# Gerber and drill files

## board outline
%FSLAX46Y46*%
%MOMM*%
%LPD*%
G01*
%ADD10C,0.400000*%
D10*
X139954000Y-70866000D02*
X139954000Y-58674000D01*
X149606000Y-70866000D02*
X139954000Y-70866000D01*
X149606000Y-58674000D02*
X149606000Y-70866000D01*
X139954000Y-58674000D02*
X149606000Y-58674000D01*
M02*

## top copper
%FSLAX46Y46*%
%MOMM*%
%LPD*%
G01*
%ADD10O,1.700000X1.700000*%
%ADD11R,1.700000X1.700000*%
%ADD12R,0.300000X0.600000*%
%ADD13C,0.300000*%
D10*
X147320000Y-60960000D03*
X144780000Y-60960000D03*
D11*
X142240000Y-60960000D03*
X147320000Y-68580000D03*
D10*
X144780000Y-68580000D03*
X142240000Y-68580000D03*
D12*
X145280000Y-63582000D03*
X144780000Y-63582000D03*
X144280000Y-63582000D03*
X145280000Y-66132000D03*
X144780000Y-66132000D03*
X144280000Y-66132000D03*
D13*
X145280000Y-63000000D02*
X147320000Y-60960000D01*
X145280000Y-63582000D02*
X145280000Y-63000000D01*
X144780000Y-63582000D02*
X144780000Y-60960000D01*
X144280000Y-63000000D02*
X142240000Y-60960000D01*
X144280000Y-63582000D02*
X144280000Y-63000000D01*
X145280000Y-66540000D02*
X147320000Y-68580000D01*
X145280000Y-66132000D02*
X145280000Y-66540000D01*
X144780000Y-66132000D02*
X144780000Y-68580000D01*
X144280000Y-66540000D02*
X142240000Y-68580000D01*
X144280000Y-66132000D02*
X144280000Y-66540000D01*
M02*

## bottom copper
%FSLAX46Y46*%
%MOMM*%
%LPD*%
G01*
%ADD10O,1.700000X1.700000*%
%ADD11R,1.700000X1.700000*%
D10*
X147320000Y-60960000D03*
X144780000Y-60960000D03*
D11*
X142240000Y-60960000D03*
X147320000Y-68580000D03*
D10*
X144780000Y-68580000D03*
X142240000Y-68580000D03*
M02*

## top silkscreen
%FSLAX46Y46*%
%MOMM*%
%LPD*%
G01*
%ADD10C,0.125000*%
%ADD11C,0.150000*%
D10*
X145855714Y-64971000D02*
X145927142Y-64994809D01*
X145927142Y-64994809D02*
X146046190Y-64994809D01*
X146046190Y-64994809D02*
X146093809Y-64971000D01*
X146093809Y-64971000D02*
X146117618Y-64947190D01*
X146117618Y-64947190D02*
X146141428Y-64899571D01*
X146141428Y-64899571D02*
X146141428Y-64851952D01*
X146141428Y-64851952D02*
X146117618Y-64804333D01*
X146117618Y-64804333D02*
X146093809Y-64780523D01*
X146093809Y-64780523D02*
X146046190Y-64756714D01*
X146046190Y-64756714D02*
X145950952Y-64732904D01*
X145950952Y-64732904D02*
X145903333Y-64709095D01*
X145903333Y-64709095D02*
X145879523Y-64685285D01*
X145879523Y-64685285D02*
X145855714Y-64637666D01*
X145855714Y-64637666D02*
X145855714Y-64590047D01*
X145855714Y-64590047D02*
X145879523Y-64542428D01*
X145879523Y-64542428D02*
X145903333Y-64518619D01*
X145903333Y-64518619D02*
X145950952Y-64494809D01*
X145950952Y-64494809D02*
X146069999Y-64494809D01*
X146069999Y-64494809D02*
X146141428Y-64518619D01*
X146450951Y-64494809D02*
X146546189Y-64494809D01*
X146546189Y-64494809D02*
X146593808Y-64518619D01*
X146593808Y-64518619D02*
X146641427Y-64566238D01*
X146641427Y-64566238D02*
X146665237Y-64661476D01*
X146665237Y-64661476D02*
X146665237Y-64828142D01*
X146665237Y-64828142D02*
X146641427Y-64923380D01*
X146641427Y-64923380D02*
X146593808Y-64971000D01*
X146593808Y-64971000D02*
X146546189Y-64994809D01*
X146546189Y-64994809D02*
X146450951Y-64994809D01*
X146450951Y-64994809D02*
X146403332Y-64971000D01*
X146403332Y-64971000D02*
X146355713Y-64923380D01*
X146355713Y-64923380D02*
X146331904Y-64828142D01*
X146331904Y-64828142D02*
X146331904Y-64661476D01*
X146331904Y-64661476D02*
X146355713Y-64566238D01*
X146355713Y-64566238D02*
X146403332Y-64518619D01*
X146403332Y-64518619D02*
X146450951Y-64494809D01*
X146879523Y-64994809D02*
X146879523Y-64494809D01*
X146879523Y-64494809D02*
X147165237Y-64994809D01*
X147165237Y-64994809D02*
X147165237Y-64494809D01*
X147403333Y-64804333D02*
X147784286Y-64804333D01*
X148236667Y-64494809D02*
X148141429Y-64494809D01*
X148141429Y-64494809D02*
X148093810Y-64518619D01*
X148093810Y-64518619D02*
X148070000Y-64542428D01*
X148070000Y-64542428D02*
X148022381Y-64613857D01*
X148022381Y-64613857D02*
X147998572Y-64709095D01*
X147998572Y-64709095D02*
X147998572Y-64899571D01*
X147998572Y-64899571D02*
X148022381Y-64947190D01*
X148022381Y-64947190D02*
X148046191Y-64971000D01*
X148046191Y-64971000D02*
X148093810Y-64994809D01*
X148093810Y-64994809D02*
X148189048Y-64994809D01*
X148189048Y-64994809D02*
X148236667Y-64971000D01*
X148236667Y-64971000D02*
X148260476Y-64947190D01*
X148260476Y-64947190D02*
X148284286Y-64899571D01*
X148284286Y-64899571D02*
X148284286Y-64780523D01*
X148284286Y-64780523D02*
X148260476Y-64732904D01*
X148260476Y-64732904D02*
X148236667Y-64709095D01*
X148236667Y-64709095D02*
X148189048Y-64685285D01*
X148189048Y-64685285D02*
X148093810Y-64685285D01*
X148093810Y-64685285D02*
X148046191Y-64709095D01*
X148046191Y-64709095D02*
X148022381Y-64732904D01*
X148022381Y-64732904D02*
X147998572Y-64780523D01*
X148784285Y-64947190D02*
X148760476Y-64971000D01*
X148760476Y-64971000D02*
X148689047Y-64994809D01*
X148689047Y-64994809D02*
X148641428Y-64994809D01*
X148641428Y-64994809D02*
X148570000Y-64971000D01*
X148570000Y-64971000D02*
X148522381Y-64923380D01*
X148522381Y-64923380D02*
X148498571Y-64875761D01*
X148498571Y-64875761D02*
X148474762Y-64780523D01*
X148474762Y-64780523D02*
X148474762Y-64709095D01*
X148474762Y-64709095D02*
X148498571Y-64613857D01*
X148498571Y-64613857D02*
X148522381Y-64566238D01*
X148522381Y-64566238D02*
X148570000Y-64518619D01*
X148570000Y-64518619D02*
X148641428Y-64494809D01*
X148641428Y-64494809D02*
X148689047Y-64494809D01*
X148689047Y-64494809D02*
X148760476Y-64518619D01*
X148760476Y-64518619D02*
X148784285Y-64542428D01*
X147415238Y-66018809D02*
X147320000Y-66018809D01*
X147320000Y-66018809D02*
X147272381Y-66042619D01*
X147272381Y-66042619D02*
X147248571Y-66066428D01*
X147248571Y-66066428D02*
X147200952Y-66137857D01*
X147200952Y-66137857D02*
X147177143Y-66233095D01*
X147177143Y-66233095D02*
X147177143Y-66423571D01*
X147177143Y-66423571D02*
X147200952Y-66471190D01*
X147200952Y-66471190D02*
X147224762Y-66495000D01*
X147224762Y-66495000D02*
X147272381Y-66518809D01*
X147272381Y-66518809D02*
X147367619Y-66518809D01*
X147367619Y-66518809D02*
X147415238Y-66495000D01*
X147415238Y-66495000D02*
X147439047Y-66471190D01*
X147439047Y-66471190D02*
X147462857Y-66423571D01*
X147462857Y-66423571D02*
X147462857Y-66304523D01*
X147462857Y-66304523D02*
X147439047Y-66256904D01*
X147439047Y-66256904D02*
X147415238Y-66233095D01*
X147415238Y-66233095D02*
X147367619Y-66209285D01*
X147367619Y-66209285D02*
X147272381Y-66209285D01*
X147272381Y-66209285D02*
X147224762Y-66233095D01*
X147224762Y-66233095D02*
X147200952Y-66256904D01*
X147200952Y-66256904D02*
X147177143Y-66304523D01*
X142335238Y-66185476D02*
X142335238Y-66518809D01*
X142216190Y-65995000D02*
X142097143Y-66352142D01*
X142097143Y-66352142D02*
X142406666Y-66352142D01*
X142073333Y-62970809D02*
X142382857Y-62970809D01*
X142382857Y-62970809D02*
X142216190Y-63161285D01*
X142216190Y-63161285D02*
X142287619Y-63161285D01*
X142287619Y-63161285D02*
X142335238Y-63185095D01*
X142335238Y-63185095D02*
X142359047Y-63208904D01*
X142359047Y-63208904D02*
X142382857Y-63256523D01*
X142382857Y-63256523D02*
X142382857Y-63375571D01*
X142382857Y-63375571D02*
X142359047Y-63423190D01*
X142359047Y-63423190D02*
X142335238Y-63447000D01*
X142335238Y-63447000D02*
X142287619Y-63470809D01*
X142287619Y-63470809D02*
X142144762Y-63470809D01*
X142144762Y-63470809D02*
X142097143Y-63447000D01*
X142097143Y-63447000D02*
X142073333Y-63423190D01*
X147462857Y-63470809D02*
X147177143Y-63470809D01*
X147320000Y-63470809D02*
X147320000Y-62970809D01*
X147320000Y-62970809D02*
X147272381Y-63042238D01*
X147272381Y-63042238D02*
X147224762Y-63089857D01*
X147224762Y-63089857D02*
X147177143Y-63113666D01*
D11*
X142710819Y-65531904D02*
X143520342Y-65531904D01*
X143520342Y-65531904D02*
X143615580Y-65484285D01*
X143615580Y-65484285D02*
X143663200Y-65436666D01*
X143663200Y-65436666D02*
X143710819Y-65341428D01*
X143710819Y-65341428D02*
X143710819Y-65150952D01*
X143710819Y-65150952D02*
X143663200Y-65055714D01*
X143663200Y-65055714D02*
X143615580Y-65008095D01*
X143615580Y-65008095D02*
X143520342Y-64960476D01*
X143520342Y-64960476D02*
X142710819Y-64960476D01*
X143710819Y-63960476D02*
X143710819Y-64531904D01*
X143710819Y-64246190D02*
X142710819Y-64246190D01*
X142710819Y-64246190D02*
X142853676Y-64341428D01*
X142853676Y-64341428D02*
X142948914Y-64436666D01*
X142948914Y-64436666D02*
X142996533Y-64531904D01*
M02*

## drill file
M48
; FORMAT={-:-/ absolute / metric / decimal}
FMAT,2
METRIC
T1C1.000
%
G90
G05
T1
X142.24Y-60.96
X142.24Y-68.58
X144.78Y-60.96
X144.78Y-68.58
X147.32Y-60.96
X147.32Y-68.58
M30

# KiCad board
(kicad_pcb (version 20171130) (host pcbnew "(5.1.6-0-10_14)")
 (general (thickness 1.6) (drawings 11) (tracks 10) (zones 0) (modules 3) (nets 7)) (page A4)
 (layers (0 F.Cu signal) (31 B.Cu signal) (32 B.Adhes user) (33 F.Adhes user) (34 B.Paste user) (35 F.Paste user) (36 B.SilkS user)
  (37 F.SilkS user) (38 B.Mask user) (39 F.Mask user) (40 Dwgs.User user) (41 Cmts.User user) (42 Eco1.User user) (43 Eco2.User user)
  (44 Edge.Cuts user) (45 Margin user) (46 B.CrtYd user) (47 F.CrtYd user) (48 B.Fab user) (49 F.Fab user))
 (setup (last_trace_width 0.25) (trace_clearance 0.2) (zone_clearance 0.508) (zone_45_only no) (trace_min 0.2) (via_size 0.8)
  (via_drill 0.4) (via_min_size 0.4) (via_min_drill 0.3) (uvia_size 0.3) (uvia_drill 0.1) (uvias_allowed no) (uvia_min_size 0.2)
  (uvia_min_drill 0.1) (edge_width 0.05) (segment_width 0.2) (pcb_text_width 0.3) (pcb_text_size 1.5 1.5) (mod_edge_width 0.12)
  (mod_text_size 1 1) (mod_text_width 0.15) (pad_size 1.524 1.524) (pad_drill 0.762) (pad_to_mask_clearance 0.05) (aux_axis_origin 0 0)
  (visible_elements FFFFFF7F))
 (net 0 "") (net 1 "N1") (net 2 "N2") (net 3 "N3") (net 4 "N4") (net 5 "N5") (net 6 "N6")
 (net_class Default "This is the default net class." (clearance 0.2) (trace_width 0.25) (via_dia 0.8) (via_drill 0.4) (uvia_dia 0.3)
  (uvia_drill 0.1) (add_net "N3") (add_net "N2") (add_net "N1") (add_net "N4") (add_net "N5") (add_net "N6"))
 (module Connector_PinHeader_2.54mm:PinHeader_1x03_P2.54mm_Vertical (layer B.Cu) (at 142.24 60.96 270)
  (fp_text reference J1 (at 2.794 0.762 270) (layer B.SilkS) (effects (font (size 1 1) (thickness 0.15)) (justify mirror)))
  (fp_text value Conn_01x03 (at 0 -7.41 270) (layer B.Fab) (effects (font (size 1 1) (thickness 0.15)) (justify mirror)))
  (pad 3 thru_hole oval (at 0 -5.08 270) (size 1.7 1.7) (drill 1) (layers *.Cu *.Mask) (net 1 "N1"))
  (pad 2 thru_hole oval (at 0 -2.54 270) (size 1.7 1.7) (drill 1) (layers *.Cu *.Mask) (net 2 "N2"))
  (pad 1 thru_hole rect (at 0 0 270) (size 1.7 1.7) (drill 1) (layers *.Cu *.Mask) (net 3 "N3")))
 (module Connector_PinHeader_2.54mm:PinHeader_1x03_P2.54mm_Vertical (layer B.Cu) (at 147.32 68.58 90)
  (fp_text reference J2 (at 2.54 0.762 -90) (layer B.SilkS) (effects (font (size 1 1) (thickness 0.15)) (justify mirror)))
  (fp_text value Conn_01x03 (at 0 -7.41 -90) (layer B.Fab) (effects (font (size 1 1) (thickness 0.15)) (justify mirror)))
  (pad 1 thru_hole rect (at 0 0 90) (size 1.7 1.7) (drill 1) (layers *.Cu *.Mask) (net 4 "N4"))
  (pad 2 thru_hole oval (at 0 -2.54 90) (size 1.7 1.7) (drill 1) (layers *.Cu *.Mask) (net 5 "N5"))
  (pad 3 thru_hole oval (at 0 -5.08 90) (size 1.7 1.7) (drill 1) (layers *.Cu *.Mask) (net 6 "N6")))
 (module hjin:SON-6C (layer F.Cu) (at 145.28 65.532 180)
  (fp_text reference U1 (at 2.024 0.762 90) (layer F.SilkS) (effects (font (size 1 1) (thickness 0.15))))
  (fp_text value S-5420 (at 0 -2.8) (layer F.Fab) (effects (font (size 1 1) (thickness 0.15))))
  (pad 1 smd rect (at 0 1.95 180) (size 0.3 0.6) (layers F.Cu F.Paste F.Mask) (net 1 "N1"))
  (pad 2 smd rect (at 0.5 1.95 180) (size 0.3 0.6) (layers F.Cu F.Paste F.Mask) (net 2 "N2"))
  (pad 3 smd rect (at 1 1.95 180) (size 0.3 0.6) (layers F.Cu F.Paste F.Mask) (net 3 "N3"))
  (pad 6 smd rect (at 0 -0.6 180) (size 0.3 0.6) (layers F.Cu F.Paste F.Mask) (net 4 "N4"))
  (pad 5 smd rect (at 0.5 -0.6 180) (size 0.3 0.6) (layers F.Cu F.Paste F.Mask) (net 5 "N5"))
  (pad 4 smd rect (at 1 -0.6 180) (size 0.3 0.6) (layers F.Cu F.Paste F.Mask) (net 6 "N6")))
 (gr_line (start 139.954 70.866) (end 139.954 58.674) (layer Edge.Cuts) (width 0.4))
 (gr_line (start 149.606 70.866) (end 139.954 70.866) (layer Edge.Cuts) (width 0.4))
 (gr_line (start 149.606 58.674) (end 149.606 70.866) (layer Edge.Cuts) (width 0.4))
 (gr_line (start 139.954 58.674) (end 149.606 58.674) (layer Edge.Cuts) (width 0.4))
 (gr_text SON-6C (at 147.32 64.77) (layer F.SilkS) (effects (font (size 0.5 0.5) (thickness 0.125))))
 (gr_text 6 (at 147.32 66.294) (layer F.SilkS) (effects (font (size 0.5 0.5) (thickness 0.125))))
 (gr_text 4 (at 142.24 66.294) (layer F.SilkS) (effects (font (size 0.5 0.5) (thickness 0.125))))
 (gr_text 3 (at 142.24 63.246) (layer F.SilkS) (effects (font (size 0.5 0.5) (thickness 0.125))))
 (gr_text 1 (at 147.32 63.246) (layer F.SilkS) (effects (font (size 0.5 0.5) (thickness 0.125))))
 (segment (start 145.28 63) (end 147.32 60.96) (width 0.3) (layer F.Cu) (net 1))
 (segment (start 145.28 63.582) (end 145.28 63) (width 0.3) (layer F.Cu) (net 1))
 (segment (start 144.78 63.582) (end 144.78 60.96) (width 0.3) (layer F.Cu) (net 2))
 (segment (start 144.28 63) (end 142.24 60.96) (width 0.3) (layer F.Cu) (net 3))
 (segment (start 144.28 63.582) (end 144.28 63) (width 0.3) (layer F.Cu) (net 3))
 (segment (start 145.28 66.54) (end 147.32 68.58) (width 0.3) (layer F.Cu) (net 4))
 (segment (start 145.28 66.132) (end 145.28 66.54) (width 0.3) (layer F.Cu) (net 4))
 (segment (start 144.78 66.132) (end 144.78 68.58) (width 0.3) (layer F.Cu) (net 5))
 (segment (start 144.28 66.54) (end 142.24 68.58) (width 0.3) (layer F.Cu) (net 6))
 (segment (start 144.28 66.132) (end 144.28 66.54) (width 0.3) (layer F.Cu) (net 6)))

